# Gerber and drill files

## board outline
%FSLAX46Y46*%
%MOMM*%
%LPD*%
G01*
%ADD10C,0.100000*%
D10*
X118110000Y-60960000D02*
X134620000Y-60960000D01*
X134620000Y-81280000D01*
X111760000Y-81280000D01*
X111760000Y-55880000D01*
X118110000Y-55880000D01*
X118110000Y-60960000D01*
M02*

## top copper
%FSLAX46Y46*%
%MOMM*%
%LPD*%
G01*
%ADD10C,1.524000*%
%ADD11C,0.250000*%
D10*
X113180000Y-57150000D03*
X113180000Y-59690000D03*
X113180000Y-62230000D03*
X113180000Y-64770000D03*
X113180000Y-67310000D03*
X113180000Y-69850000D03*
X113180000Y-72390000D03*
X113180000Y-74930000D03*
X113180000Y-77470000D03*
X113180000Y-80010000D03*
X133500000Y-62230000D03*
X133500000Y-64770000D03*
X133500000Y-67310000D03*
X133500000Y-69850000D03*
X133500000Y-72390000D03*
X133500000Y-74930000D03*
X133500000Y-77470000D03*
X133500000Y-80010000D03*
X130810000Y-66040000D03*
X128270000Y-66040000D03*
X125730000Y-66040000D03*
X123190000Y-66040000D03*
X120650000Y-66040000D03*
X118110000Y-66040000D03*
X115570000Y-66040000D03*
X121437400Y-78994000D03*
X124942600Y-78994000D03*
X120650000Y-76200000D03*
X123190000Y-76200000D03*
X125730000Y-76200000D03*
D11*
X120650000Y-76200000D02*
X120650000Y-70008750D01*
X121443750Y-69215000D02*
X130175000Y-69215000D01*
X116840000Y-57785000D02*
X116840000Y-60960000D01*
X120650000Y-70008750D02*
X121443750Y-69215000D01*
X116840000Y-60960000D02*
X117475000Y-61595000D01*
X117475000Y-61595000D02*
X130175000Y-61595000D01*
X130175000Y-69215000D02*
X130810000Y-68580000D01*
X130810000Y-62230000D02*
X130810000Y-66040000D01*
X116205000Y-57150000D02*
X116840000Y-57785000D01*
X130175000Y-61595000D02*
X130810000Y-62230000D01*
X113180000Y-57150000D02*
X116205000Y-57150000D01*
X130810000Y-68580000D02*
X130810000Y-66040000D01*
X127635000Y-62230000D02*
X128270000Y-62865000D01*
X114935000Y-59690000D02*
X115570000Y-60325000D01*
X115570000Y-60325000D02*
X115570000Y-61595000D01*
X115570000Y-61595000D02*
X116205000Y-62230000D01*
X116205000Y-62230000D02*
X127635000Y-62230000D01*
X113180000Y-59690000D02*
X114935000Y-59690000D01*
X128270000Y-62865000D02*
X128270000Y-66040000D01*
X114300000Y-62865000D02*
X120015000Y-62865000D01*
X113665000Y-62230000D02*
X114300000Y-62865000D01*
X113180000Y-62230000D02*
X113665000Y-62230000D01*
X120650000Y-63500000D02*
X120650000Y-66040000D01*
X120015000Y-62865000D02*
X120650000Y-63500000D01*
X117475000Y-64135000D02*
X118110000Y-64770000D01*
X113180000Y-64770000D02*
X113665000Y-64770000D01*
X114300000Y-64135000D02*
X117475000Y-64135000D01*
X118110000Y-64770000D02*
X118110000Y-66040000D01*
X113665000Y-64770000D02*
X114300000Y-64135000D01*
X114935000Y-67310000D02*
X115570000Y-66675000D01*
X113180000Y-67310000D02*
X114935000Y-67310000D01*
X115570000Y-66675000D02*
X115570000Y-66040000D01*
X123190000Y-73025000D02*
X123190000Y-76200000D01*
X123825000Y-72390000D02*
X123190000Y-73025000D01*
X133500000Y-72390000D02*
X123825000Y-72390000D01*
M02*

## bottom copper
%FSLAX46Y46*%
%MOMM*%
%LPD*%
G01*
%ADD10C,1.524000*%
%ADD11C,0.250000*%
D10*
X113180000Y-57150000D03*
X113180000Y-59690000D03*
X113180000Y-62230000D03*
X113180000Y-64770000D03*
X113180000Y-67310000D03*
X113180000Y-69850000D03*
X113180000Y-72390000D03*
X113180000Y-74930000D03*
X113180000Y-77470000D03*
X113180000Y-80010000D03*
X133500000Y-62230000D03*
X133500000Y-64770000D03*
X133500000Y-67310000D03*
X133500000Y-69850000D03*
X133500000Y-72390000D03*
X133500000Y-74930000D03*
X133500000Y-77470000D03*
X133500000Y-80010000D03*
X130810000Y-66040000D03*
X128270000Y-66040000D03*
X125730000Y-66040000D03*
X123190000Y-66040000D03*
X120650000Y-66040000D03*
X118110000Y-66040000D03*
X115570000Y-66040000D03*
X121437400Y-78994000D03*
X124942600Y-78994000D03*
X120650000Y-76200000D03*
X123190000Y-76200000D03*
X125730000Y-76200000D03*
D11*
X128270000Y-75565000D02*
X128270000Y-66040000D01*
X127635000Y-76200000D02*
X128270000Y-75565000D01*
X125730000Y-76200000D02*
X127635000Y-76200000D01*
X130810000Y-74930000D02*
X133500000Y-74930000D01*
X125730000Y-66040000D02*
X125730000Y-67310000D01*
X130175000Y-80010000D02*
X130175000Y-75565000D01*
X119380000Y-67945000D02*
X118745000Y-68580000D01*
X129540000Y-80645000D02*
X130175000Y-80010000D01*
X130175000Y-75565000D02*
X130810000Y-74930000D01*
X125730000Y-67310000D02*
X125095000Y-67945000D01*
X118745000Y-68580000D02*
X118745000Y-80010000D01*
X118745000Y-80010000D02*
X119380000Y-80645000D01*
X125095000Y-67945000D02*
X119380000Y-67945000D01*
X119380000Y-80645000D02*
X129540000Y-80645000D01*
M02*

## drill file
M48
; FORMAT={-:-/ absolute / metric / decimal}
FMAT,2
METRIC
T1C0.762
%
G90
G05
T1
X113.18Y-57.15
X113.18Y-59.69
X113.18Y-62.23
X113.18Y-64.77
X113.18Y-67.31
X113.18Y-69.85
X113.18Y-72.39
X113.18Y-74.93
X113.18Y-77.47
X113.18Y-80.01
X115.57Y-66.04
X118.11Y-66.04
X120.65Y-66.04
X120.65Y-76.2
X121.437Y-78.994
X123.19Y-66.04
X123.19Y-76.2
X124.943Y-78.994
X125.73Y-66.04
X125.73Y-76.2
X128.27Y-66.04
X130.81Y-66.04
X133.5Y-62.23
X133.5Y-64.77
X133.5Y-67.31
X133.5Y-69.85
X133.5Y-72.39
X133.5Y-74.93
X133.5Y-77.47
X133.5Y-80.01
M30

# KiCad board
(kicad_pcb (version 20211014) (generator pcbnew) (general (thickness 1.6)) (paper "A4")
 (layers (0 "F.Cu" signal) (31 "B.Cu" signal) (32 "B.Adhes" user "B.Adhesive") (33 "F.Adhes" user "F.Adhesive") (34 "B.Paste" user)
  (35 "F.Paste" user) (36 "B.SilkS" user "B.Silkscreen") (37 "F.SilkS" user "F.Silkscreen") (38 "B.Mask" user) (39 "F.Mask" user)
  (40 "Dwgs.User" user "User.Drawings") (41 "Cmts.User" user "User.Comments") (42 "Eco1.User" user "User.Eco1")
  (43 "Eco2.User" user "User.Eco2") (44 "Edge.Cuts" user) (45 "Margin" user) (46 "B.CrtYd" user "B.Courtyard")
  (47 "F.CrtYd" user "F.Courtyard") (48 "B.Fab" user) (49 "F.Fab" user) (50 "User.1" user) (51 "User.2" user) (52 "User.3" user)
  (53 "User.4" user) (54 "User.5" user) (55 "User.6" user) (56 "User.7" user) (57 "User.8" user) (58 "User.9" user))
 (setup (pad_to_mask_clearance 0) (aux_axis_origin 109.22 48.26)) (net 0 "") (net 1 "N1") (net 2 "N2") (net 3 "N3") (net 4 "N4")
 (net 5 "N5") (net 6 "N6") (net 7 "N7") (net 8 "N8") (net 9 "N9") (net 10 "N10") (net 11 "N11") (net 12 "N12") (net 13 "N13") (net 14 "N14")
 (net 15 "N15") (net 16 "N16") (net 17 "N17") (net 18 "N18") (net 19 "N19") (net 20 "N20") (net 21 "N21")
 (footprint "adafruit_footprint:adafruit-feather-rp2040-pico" (layer "F.Cu") (at 123.34 80.01)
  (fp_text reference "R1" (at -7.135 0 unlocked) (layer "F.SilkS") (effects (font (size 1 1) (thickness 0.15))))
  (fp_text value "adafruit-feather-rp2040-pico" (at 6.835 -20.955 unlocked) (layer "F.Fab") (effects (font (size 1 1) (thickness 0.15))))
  (pad "3" thru_hole circle (at -10.16 -22.86) (size 1.524 1.524) (drill 0.762) (layers *.Cu *.Mask) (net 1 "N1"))
  (pad "4" thru_hole circle (at -10.16 -20.32) (size 1.524 1.524) (drill 0.762) (layers *.Cu *.Mask) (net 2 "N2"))
  (pad "5" thru_hole circle (at -10.16 -17.78) (size 1.524 1.524) (drill 0.762) (layers *.Cu *.Mask) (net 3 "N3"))
  (pad "6" thru_hole circle (at -10.16 -15.24) (size 1.524 1.524) (drill 0.762) (layers *.Cu *.Mask) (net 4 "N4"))
  (pad "7" thru_hole circle (at -10.16 -12.7) (size 1.524 1.524) (drill 0.762) (layers *.Cu *.Mask) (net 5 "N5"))
  (pad "8" thru_hole circle (at -10.16 -10.16) (size 1.524 1.524) (drill 0.762) (layers *.Cu *.Mask) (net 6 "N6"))
  (pad "9" thru_hole circle (at -10.16 -7.62) (size 1.524 1.524) (drill 0.762) (layers *.Cu *.Mask) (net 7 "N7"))
  (pad "10" thru_hole circle (at -10.16 -5.08) (size 1.524 1.524) (drill 0.762) (layers *.Cu *.Mask) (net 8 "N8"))
  (pad "11" thru_hole circle (at -10.16 -2.54) (size 1.524 1.524) (drill 0.762) (layers *.Cu *.Mask) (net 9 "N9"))
  (pad "12" thru_hole circle (at -10.16 0) (size 1.524 1.524) (drill 0.762) (layers *.Cu *.Mask) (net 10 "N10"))
  (pad "17" thru_hole circle (at 10.16 -17.78) (size 1.524 1.524) (drill 0.762) (layers *.Cu *.Mask) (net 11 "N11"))
  (pad "18" thru_hole circle (at 10.16 -15.24) (size 1.524 1.524) (drill 0.762) (layers *.Cu *.Mask) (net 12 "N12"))
  (pad "19" thru_hole circle (at 10.16 -12.7) (size 1.524 1.524) (drill 0.762) (layers *.Cu *.Mask) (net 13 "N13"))
  (pad "20" thru_hole circle (at 10.16 -10.16) (size 1.524 1.524) (drill 0.762) (layers *.Cu *.Mask) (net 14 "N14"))
  (pad "21" thru_hole circle (at 10.16 -7.62) (size 1.524 1.524) (drill 0.762) (layers *.Cu *.Mask) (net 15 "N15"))
  (pad "22" thru_hole circle (at 10.16 -5.08) (size 1.524 1.524) (drill 0.762) (layers *.Cu *.Mask) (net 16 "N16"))
  (pad "23" thru_hole circle (at 10.16 -2.54) (size 1.524 1.524) (drill 0.762) (layers *.Cu *.Mask) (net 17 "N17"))
  (pad "24" thru_hole circle (at 10.16 0) (size 1.524 1.524) (drill 0.762) (layers *.Cu *.Mask) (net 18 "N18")))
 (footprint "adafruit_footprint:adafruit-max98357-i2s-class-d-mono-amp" (layer "B.Cu") (at 123.19 73.66)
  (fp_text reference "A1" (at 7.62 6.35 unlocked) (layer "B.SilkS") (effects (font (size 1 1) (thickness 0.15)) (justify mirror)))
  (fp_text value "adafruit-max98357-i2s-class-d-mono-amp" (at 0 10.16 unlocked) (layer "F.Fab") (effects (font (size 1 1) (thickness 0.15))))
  (pad "1" thru_hole circle (at 7.62 -7.62) (size 1.524 1.524) (drill 0.762) (layers *.Cu *.Mask) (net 1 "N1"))
  (pad "2" thru_hole circle (at 5.08 -7.62) (size 1.524 1.524) (drill 0.762) (layers *.Cu *.Mask) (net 2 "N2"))
  (pad "3" thru_hole circle (at 2.54 -7.62) (size 1.524 1.524) (drill 0.762) (layers *.Cu *.Mask) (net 16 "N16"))
  (pad "4" thru_hole circle (at 0 -7.62) (size 1.524 1.524) (drill 0.762) (layers *.Cu *.Mask) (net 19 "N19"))
  (pad "5" thru_hole circle (at -2.54 -7.62) (size 1.524 1.524) (drill 0.762) (layers *.Cu *.Mask) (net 3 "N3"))
  (pad "6" thru_hole circle (at -5.08 -7.62) (size 1.524 1.524) (drill 0.762) (layers *.Cu *.Mask) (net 4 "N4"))
  (pad "7" thru_hole circle (at -7.62 -7.62) (size 1.524 1.524) (drill 0.762) (layers *.Cu *.Mask) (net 5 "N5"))
  (pad "8" thru_hole circle (at -1.7526 5.334) (size 1.524 1.524) (drill 0.762) (layers *.Cu *.Mask) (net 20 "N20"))
  (pad "9" thru_hole circle (at 1.7526 5.334) (size 1.524 1.524) (drill 0.762) (layers *.Cu *.Mask) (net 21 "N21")))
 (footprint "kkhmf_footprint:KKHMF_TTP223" (layer "B.Cu") (at 123.19 73.66 180)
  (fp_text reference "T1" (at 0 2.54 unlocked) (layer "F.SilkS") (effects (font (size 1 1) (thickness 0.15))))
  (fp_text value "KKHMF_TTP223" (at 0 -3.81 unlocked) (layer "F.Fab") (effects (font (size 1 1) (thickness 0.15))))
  (pad "1" thru_hole circle (at 2.54 -2.54 180) (size 1.524 1.524) (drill 0.762) (layers *.Cu *.Mask) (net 1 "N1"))
  (pad "2" thru_hole circle (at 0 -2.54 180) (size 1.524 1.524) (drill 0.762) (layers *.Cu *.Mask) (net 15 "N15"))
  (pad "3" thru_hole circle (at -2.54 -2.54 180) (size 1.524 1.524) (drill 0.762) (layers *.Cu *.Mask) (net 2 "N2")))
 (gr_poly
  (pts (xy 118.11 60.96) (xy 134.62 60.96) (xy 134.62 81.28) (xy 111.76 81.28) (xy 111.76 55.88) (xy 118.11 55.88)) (layer "Edge.Cuts")
  (width 0.1) (fill none))
 (segment (start 120.65 76.2) (end 120.65 70.00875) (width 0.25) (layer "F.Cu") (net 1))
 (segment (start 121.44375 69.215) (end 130.175 69.215) (width 0.25) (layer "F.Cu") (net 1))
 (segment (start 116.84 57.785) (end 116.84 60.96) (width 0.25) (layer "F.Cu") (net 1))
 (segment (start 120.65 70.00875) (end 121.44375 69.215) (width 0.25) (layer "F.Cu") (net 1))
 (segment (start 116.84 60.96) (end 117.475 61.595) (width 0.25) (layer "F.Cu") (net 1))
 (segment (start 117.475 61.595) (end 130.175 61.595) (width 0.25) (layer "F.Cu") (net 1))
 (segment (start 130.175 69.215) (end 130.81 68.58) (width 0.25) (layer "F.Cu") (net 1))
 (segment (start 130.81 62.23) (end 130.81 66.04) (width 0.25) (layer "F.Cu") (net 1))
 (segment (start 116.205 57.15) (end 116.84 57.785) (width 0.25) (layer "F.Cu") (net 1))
 (segment (start 130.175 61.595) (end 130.81 62.23) (width 0.25) (layer "F.Cu") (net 1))
 (segment (start 113.18 57.15) (end 116.205 57.15) (width 0.25) (layer "F.Cu") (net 1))
 (segment (start 130.81 68.58) (end 130.81 66.04) (width 0.25) (layer "F.Cu") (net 1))
 (segment (start 127.635 62.23) (end 128.27 62.865) (width 0.25) (layer "F.Cu") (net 2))
 (segment (start 114.935 59.69) (end 115.57 60.325) (width 0.25) (layer "F.Cu") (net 2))
 (segment (start 115.57 60.325) (end 115.57 61.595) (width 0.25) (layer "F.Cu") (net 2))
 (segment (start 115.57 61.595) (end 116.205 62.23) (width 0.25) (layer "F.Cu") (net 2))
 (segment (start 116.205 62.23) (end 127.635 62.23) (width 0.25) (layer "F.Cu") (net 2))
 (segment (start 113.18 59.69) (end 114.935 59.69) (width 0.25) (layer "F.Cu") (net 2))
 (segment (start 128.27 62.865) (end 128.27 66.04) (width 0.25) (layer "F.Cu") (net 2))
 (segment (start 128.27 75.565) (end 128.27 66.04) (width 0.25) (layer "B.Cu") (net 2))
 (segment (start 127.635 76.2) (end 128.27 75.565) (width 0.25) (layer "B.Cu") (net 2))
 (segment (start 125.73 76.2) (end 127.635 76.2) (width 0.25) (layer "B.Cu") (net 2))
 (segment (start 130.81 74.93) (end 133.5 74.93) (width 0.25) (layer "B.Cu") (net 16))
 (segment (start 125.73 66.04) (end 125.73 67.31) (width 0.25) (layer "B.Cu") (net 16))
 (segment (start 130.175 80.01) (end 130.175 75.565) (width 0.25) (layer "B.Cu") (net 16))
 (segment (start 119.38 67.945) (end 118.745 68.58) (width 0.25) (layer "B.Cu") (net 16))
 (segment (start 129.54 80.645) (end 130.175 80.01) (width 0.25) (layer "B.Cu") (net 16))
 (segment (start 130.175 75.565) (end 130.81 74.93) (width 0.25) (layer "B.Cu") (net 16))
 (segment (start 125.73 67.31) (end 125.095 67.945) (width 0.25) (layer "B.Cu") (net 16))
 (segment (start 118.745 68.58) (end 118.745 80.01) (width 0.25) (layer "B.Cu") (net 16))
 (segment (start 118.745 80.01) (end 119.38 80.645) (width 0.25) (layer "B.Cu") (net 16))
 (segment (start 125.095 67.945) (end 119.38 67.945) (width 0.25) (layer "B.Cu") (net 16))
 (segment (start 119.38 80.645) (end 129.54 80.645) (width 0.25) (layer "B.Cu") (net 16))
 (segment (start 114.3 62.865) (end 120.015 62.865) (width 0.25) (layer "F.Cu") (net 3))
 (segment (start 113.665 62.23) (end 114.3 62.865) (width 0.25) (layer "F.Cu") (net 3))
 (segment (start 113.18 62.23) (end 113.665 62.23) (width 0.25) (layer "F.Cu") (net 3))
 (segment (start 120.65 63.5) (end 120.65 66.04) (width 0.25) (layer "F.Cu") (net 3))
 (segment (start 120.015 62.865) (end 120.65 63.5) (width 0.25) (layer "F.Cu") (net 3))
 (segment (start 117.475 64.135) (end 118.11 64.77) (width 0.25) (layer "F.Cu") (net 4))
 (segment (start 113.18 64.77) (end 113.665 64.77) (width 0.25) (layer "F.Cu") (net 4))
 (segment (start 114.3 64.135) (end 117.475 64.135) (width 0.25) (layer "F.Cu") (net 4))
 (segment (start 118.11 64.77) (end 118.11 66.04) (width 0.25) (layer "F.Cu") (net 4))
 (segment (start 113.665 64.77) (end 114.3 64.135) (width 0.25) (layer "F.Cu") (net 4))
 (segment (start 114.935 67.31) (end 115.57 66.675) (width 0.25) (layer "F.Cu") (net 5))
 (segment (start 113.18 67.31) (end 114.935 67.31) (width 0.25) (layer "F.Cu") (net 5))
 (segment (start 115.57 66.675) (end 115.57 66.04) (width 0.25) (layer "F.Cu") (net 5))
 (segment (start 123.19 73.025) (end 123.19 76.2) (width 0.25) (layer "F.Cu") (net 15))
 (segment (start 123.825 72.39) (end 123.19 73.025) (width 0.25) (layer "F.Cu") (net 15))
 (segment (start 133.5 72.39) (end 123.825 72.39) (width 0.25) (layer "F.Cu") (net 15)))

